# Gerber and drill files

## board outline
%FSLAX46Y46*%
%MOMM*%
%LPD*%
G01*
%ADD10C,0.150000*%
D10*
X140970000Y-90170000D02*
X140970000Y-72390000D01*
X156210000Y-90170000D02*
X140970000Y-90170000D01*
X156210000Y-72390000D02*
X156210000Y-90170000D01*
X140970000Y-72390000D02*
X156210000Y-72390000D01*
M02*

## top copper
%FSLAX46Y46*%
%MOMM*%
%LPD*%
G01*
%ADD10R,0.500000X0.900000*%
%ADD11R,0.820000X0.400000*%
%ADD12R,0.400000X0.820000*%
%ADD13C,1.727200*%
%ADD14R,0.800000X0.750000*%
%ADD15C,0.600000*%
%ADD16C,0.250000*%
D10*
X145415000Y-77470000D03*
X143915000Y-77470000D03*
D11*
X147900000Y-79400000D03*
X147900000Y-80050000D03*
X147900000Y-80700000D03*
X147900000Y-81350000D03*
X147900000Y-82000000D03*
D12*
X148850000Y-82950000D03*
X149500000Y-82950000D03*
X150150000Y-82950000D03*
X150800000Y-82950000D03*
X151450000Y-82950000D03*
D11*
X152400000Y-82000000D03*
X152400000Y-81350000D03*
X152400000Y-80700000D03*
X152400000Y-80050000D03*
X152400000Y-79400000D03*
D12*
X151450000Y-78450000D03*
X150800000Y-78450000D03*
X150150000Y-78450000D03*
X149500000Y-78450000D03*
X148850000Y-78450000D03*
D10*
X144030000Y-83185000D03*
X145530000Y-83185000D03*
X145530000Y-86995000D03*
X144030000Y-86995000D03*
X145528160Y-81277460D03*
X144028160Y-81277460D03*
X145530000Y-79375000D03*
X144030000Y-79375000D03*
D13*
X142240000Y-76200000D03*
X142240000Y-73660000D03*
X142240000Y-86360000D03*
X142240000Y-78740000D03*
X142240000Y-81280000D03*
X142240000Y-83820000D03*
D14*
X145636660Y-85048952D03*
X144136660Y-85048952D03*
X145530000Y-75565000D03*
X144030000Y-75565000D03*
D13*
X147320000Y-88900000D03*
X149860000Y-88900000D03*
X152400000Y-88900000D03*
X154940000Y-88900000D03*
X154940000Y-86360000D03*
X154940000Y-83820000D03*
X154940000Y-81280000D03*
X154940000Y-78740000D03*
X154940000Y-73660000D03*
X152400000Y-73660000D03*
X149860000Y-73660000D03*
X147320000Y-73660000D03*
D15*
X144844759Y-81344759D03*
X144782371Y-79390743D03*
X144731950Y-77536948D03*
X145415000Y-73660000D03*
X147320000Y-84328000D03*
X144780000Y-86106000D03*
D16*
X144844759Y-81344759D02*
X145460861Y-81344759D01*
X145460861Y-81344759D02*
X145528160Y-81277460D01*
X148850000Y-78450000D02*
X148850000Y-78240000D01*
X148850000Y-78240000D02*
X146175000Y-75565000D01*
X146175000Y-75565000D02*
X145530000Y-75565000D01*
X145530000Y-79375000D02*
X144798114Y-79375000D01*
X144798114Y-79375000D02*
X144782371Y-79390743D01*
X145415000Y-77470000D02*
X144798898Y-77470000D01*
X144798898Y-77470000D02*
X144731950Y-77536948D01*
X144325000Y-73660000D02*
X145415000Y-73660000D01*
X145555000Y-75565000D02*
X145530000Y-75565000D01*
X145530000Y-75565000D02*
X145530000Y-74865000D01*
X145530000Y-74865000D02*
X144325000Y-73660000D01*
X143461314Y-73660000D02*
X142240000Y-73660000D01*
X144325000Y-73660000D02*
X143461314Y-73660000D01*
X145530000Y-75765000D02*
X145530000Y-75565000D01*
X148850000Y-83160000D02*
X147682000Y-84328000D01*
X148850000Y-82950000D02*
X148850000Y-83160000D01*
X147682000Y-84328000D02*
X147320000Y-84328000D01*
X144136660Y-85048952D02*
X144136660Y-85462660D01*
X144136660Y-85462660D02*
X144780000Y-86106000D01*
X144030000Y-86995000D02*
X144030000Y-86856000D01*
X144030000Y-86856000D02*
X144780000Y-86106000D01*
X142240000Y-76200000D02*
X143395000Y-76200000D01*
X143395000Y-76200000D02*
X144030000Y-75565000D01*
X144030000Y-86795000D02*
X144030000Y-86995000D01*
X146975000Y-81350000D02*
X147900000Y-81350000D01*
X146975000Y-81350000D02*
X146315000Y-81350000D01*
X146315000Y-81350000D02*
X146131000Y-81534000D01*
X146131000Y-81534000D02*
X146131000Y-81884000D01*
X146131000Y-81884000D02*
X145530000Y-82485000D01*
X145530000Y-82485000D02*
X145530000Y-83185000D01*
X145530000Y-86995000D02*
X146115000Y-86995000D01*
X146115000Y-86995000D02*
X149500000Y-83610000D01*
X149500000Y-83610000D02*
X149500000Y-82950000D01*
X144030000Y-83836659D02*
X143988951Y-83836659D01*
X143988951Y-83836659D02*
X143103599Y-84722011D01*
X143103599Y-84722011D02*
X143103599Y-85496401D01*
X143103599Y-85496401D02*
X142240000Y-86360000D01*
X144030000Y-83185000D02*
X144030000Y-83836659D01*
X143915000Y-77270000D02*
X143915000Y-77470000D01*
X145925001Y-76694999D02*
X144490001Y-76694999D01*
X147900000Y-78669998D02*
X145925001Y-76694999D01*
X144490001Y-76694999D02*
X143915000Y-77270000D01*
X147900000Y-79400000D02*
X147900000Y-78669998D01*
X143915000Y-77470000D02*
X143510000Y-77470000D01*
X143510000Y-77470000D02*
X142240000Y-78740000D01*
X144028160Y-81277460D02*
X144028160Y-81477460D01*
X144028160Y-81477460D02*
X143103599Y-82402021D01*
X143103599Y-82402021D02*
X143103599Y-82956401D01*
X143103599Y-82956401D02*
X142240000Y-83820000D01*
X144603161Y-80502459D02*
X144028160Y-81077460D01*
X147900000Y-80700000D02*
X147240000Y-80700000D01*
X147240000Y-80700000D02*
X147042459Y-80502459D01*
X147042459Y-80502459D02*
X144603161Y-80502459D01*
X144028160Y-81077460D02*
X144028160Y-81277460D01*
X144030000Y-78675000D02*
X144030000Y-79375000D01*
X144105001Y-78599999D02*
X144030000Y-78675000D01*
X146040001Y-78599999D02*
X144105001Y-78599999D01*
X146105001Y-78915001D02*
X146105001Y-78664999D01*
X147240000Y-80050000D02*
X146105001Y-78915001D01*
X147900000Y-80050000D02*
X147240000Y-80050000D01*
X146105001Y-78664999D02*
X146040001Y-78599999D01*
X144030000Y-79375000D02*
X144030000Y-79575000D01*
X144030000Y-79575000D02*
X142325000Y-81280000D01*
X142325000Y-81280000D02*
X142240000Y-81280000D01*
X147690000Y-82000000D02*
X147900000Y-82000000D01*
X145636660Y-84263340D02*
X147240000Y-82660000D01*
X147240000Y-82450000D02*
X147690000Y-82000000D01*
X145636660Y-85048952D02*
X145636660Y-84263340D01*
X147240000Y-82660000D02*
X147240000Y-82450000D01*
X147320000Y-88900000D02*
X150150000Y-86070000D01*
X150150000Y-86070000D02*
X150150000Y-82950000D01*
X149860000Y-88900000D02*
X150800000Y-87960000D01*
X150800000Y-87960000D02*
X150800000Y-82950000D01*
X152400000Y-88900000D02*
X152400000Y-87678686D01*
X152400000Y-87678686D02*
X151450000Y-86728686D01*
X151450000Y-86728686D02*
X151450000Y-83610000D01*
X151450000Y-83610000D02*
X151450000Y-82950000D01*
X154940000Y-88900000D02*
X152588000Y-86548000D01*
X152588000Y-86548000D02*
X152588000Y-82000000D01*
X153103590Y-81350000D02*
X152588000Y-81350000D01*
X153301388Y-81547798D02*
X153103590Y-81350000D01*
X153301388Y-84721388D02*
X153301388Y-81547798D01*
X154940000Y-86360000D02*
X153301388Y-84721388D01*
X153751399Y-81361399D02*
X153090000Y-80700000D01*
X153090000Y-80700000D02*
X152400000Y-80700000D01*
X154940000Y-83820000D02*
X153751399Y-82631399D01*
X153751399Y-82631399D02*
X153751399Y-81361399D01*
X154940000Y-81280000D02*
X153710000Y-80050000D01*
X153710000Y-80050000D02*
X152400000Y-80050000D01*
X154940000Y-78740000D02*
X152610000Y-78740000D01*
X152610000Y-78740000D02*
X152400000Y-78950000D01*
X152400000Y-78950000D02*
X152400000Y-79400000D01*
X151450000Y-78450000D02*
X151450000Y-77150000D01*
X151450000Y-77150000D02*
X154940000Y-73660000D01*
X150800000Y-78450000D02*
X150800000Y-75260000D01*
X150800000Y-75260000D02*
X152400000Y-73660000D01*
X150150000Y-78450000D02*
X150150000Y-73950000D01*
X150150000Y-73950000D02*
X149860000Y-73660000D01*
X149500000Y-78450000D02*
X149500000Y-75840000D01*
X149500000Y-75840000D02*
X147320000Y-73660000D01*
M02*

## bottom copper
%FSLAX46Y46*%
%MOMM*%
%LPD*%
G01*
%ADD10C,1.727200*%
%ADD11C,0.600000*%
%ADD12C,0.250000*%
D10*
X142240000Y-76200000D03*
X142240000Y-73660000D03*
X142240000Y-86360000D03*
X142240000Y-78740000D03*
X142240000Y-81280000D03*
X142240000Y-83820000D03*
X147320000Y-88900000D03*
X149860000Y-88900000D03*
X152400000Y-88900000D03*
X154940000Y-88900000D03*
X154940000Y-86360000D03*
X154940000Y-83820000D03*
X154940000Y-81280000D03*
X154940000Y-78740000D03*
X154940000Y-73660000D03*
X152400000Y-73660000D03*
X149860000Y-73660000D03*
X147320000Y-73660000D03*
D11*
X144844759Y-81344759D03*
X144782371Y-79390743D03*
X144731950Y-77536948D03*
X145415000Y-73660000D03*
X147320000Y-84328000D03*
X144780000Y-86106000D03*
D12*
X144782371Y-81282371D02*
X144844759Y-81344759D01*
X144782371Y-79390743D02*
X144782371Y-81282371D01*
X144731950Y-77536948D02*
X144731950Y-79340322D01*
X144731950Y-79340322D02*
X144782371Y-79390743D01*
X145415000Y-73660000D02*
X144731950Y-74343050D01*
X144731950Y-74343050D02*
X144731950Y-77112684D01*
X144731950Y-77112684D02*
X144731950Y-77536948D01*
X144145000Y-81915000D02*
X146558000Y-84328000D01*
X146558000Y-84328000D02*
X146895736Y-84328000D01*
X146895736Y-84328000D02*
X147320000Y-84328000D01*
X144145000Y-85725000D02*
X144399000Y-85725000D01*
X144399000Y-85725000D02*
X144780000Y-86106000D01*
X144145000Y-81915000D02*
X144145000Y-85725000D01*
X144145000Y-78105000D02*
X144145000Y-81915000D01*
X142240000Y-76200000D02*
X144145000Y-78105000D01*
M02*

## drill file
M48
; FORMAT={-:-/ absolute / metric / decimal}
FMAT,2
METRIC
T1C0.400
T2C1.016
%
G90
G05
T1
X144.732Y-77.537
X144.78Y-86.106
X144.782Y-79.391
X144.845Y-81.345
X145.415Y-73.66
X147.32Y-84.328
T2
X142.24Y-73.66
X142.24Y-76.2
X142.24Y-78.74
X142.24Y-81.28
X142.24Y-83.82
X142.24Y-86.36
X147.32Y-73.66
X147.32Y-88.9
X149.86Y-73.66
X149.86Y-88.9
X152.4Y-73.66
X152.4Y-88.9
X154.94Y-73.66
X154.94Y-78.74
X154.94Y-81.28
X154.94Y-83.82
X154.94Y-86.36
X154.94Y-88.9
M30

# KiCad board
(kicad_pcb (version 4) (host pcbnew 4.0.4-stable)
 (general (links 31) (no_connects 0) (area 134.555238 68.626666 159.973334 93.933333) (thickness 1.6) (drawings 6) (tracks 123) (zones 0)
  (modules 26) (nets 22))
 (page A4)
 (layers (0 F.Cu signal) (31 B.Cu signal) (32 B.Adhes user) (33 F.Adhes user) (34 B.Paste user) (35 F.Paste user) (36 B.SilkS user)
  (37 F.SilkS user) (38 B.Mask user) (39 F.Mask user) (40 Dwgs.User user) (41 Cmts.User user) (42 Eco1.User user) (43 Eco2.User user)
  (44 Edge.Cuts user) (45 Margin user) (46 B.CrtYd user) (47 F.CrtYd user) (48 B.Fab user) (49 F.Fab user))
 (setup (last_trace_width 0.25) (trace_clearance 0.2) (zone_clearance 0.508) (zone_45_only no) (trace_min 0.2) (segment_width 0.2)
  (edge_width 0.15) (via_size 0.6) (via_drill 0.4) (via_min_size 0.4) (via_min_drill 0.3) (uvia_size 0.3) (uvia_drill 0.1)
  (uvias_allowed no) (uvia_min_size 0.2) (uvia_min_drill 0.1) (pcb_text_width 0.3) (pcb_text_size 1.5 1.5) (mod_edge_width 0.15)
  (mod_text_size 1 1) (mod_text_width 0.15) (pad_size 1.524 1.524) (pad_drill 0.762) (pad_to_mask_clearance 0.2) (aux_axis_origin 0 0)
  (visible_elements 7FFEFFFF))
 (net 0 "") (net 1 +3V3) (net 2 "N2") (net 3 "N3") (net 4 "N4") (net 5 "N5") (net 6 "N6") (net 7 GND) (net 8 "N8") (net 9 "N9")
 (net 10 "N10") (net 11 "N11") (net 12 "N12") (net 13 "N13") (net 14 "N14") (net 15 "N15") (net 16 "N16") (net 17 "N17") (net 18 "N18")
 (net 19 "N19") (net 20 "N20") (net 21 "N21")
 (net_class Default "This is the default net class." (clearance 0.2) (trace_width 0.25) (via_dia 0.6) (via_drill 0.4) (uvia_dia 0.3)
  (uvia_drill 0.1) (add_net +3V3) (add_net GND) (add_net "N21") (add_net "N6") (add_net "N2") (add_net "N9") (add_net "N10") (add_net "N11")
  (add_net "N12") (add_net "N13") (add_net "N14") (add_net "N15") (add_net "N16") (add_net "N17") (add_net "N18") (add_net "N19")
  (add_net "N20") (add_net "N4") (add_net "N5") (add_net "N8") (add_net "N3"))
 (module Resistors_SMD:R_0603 (layer F.Cu) (at 144.665 77.47 180)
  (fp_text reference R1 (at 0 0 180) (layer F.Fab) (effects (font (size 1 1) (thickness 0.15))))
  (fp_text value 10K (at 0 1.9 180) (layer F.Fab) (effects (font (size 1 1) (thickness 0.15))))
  (pad 1 smd rect (at -0.75 0 180) (size 0.5 0.9) (layers F.Cu F.Paste F.Mask) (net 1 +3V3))
  (pad 2 smd rect (at 0.75 0 180) (size 0.5 0.9) (layers F.Cu F.Paste F.Mask) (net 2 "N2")))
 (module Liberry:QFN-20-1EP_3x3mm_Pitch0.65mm (layer F.Cu) (at 150.15 80.7)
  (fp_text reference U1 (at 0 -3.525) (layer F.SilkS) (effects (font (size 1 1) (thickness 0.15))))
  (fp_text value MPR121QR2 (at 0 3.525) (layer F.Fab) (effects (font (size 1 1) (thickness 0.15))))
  (pad 1 smd rect (at -2.25 -1.3) (size 0.82 0.4) (layers F.Cu F.Paste F.Mask) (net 2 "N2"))
  (pad 2 smd rect (at -2.25 -0.65) (size 0.82 0.4) (layers F.Cu F.Paste F.Mask) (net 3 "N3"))
  (pad 3 smd rect (at -2.25 0) (size 0.82 0.4) (layers F.Cu F.Paste F.Mask) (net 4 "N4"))
  (pad 4 smd rect (at -2.25 0.65) (size 0.82 0.4) (layers F.Cu F.Paste F.Mask) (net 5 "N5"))
  (pad 5 smd rect (at -2.25 1.3) (size 0.82 0.4) (layers F.Cu F.Paste F.Mask) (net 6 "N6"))
  (pad 6 smd rect (at -1.3 2.25 90) (size 0.82 0.4) (layers F.Cu F.Paste F.Mask) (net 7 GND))
  (pad 7 smd rect (at -0.65 2.25 90) (size 0.82 0.4) (layers F.Cu F.Paste F.Mask) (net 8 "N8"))
  (pad 8 smd rect (at 0 2.25 90) (size 0.82 0.4) (layers F.Cu F.Paste F.Mask) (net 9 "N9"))
  (pad 9 smd rect (at 0.65 2.25 90) (size 0.82 0.4) (layers F.Cu F.Paste F.Mask) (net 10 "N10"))
  (pad 10 smd rect (at 1.3 2.25 90) (size 0.82 0.4) (layers F.Cu F.Paste F.Mask) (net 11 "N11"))
  (pad 11 smd rect (at 2.25 1.3) (size 0.82 0.4) (layers F.Cu F.Paste F.Mask) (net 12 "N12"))
  (pad 12 smd rect (at 2.25 0.65) (size 0.82 0.4) (layers F.Cu F.Paste F.Mask) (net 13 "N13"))
  (pad 13 smd rect (at 2.25 0) (size 0.82 0.4) (layers F.Cu F.Paste F.Mask) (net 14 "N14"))
  (pad 14 smd rect (at 2.25 -0.65) (size 0.82 0.4) (layers F.Cu F.Paste F.Mask) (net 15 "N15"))
  (pad 15 smd rect (at 2.25 -1.3) (size 0.82 0.4) (layers F.Cu F.Paste F.Mask) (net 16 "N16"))
  (pad 16 smd rect (at 1.3 -2.25 90) (size 0.82 0.4) (layers F.Cu F.Paste F.Mask) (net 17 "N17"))
  (pad 17 smd rect (at 0.65 -2.25 90) (size 0.82 0.4) (layers F.Cu F.Paste F.Mask) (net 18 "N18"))
  (pad 18 smd rect (at 0 -2.25 90) (size 0.82 0.4) (layers F.Cu F.Paste F.Mask) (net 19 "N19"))
  (pad 19 smd rect (at -0.65 -2.25 90) (size 0.82 0.4) (layers F.Cu F.Paste F.Mask) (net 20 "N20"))
  (pad 20 smd rect (at -1.3 -2.25 90) (size 0.82 0.4) (layers F.Cu F.Paste F.Mask) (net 1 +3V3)))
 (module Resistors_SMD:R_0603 (layer F.Cu) (at 144.78 83.185)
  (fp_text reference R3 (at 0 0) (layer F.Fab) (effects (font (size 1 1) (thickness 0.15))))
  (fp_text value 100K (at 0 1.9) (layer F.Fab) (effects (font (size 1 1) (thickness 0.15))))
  (pad 1 smd rect (at -0.75 0) (size 0.5 0.9) (layers F.Cu F.Paste F.Mask) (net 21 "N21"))
  (pad 2 smd rect (at 0.75 0) (size 0.5 0.9) (layers F.Cu F.Paste F.Mask) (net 5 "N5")))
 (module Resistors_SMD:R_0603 (layer F.Cu) (at 144.78 86.995 180)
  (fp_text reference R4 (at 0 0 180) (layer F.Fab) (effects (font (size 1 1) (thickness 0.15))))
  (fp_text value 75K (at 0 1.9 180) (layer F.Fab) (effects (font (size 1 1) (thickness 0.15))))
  (pad 1 smd rect (at -0.75 0 180) (size 0.5 0.9) (layers F.Cu F.Paste F.Mask) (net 8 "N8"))
  (pad 2 smd rect (at 0.75 0 180) (size 0.5 0.9) (layers F.Cu F.Paste F.Mask) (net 7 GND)))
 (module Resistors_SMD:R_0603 (layer F.Cu) (at 144.77816 81.27746 180)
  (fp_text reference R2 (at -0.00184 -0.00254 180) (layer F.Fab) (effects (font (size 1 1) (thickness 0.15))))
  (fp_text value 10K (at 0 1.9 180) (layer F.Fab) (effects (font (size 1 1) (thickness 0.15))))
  (pad 1 smd rect (at -0.75 0 180) (size 0.5 0.9) (layers F.Cu F.Paste F.Mask) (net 1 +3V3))
  (pad 2 smd rect (at 0.75 0 180) (size 0.5 0.9) (layers F.Cu F.Paste F.Mask) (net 4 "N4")))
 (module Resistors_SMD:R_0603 (layer F.Cu) (at 144.78 79.375 180)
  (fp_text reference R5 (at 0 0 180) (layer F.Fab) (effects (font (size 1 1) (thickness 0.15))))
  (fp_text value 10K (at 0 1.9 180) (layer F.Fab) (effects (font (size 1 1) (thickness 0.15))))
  (pad 1 smd rect (at -0.75 0 180) (size 0.5 0.9) (layers F.Cu F.Paste F.Mask) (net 1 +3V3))
  (pad 2 smd rect (at 0.75 0 180) (size 0.5 0.9) (layers F.Cu F.Paste F.Mask) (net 3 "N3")))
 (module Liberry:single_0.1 (layer F.Cu) (at 142.24 76.2)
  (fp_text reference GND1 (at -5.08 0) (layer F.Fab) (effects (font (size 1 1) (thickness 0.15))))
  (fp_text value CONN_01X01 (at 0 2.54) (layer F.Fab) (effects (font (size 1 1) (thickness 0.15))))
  (pad 1 thru_hole circle (at 0 0) (size 1.7272 1.7272) (drill 1.016) (layers *.Cu *.Mask) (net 7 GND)))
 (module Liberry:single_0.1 (layer F.Cu) (at 142.24 73.66)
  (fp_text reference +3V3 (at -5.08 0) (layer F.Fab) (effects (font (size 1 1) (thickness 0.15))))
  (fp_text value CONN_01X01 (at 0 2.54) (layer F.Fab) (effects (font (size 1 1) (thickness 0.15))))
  (pad 1 thru_hole circle (at 0 0) (size 1.7272 1.7272) (drill 1.016) (layers *.Cu *.Mask) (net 1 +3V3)))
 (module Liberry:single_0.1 (layer F.Cu) (at 142.24 86.36)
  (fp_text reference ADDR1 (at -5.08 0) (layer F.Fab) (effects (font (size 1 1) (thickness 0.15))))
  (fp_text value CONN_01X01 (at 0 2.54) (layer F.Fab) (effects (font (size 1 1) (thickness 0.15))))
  (pad 1 thru_hole circle (at 0 0) (size 1.7272 1.7272) (drill 1.016) (layers *.Cu *.Mask) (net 21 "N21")))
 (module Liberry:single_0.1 (layer F.Cu) (at 142.24 78.74)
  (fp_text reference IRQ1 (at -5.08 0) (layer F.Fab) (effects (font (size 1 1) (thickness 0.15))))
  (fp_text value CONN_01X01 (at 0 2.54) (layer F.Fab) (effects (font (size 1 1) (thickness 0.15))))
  (pad 1 thru_hole circle (at 0 0) (size 1.7272 1.7272) (drill 1.016) (layers *.Cu *.Mask) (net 2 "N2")))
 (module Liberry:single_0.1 (layer F.Cu) (at 142.24 81.28)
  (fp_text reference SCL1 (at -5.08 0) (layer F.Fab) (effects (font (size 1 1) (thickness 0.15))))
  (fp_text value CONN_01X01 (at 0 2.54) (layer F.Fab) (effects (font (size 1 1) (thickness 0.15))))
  (pad 1 thru_hole circle (at 0 0) (size 1.7272 1.7272) (drill 1.016) (layers *.Cu *.Mask) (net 3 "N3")))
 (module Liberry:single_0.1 (layer F.Cu) (at 142.24 83.82)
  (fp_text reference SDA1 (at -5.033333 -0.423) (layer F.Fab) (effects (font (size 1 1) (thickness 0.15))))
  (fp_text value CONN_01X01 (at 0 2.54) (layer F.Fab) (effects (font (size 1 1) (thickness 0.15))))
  (pad 1 thru_hole circle (at 0 0) (size 1.7272 1.7272) (drill 1.016) (layers *.Cu *.Mask) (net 4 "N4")))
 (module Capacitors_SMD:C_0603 (layer F.Cu) (at 144.88666 85.048952 180)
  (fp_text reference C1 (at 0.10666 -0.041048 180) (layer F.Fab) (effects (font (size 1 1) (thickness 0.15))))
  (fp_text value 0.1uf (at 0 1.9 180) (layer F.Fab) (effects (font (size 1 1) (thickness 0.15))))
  (pad 1 smd rect (at -0.75 0 180) (size 0.8 0.75) (layers F.Cu F.Paste F.Mask) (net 6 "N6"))
  (pad 2 smd rect (at 0.75 0 180) (size 0.8 0.75) (layers F.Cu F.Paste F.Mask) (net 7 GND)))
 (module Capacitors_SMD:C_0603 (layer F.Cu) (at 144.78 75.565 180)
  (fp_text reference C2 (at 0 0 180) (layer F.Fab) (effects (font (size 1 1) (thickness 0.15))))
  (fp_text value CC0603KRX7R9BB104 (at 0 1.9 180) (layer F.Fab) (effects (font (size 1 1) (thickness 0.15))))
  (pad 1 smd rect (at -0.75 0 180) (size 0.8 0.75) (layers F.Cu F.Paste F.Mask) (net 1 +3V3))
  (pad 2 smd rect (at 0.75 0 180) (size 0.8 0.75) (layers F.Cu F.Paste F.Mask) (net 7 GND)))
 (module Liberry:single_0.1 (layer F.Cu) (at 147.32 88.9 270)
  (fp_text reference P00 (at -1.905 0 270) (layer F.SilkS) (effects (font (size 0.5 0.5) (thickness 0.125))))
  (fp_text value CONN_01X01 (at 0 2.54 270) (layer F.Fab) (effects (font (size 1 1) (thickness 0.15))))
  (pad 1 thru_hole circle (at 0 0 270) (size 1.7272 1.7272) (drill 1.016) (layers *.Cu *.Mask) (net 9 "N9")))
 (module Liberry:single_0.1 (layer F.Cu) (at 149.86 88.9 270)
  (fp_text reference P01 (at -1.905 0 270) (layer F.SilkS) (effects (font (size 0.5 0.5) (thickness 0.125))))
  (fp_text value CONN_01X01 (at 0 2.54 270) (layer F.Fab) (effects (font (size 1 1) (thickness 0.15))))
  (pad 1 thru_hole circle (at 0 0 270) (size 1.7272 1.7272) (drill 1.016) (layers *.Cu *.Mask) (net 10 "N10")))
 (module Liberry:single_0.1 (layer F.Cu) (at 152.4 88.9 270)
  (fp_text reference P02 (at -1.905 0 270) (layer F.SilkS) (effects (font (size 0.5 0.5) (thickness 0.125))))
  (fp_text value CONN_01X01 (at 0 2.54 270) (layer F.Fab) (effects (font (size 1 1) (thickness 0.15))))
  (pad 1 thru_hole circle (at 0 0 270) (size 1.7272 1.7272) (drill 1.016) (layers *.Cu *.Mask) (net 11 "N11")))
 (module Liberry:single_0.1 (layer F.Cu) (at 154.94 88.9 270)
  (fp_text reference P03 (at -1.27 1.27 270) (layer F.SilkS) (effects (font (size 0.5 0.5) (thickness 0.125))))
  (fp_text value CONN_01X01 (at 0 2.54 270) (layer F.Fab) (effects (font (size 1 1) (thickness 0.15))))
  (pad 1 thru_hole circle (at 0 0 270) (size 1.7272 1.7272) (drill 1.016) (layers *.Cu *.Mask) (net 12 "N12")))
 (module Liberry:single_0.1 (layer F.Cu) (at 154.94 86.36)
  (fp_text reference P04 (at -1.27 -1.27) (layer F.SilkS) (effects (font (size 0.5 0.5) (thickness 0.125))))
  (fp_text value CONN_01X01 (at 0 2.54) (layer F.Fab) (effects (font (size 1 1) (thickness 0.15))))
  (pad 1 thru_hole circle (at 0 0) (size 1.7272 1.7272) (drill 1.016) (layers *.Cu *.Mask) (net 13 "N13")))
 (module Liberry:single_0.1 (layer F.Cu) (at 154.94 83.82)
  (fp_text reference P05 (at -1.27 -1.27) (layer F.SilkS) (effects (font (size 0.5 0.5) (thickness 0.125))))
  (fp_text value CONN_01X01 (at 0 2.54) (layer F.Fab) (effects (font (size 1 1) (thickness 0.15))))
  (pad 1 thru_hole circle (at 0 0) (size 1.7272 1.7272) (drill 1.016) (layers *.Cu *.Mask) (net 14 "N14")))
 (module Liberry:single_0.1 (layer F.Cu) (at 154.94 81.28)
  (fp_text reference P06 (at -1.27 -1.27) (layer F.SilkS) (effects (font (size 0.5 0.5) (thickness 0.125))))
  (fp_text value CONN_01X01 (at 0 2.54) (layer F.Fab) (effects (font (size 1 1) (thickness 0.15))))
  (pad 1 thru_hole circle (at 0 0) (size 1.7272 1.7272) (drill 1.016) (layers *.Cu *.Mask) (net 15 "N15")))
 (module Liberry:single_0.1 (layer F.Cu) (at 154.94 78.74)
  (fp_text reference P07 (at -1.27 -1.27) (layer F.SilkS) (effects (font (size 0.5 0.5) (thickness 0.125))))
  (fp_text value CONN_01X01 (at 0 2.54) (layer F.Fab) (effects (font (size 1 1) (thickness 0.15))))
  (pad 1 thru_hole circle (at 0 0) (size 1.7272 1.7272) (drill 1.016) (layers *.Cu *.Mask) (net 16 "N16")))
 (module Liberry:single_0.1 (layer F.Cu) (at 154.94 73.66 90)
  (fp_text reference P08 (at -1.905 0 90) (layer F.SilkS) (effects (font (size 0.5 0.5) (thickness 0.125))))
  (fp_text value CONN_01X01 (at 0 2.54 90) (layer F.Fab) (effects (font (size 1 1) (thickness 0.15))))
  (pad 1 thru_hole circle (at 0 0 90) (size 1.7272 1.7272) (drill 1.016) (layers *.Cu *.Mask) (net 17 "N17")))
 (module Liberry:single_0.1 (layer F.Cu) (at 152.4 73.66 90)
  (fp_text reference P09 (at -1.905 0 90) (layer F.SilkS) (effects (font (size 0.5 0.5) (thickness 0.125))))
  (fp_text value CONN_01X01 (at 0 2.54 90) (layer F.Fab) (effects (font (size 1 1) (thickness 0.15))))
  (pad 1 thru_hole circle (at 0 0 90) (size 1.7272 1.7272) (drill 1.016) (layers *.Cu *.Mask) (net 18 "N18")))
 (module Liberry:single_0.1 (layer F.Cu) (at 149.86 73.66 90)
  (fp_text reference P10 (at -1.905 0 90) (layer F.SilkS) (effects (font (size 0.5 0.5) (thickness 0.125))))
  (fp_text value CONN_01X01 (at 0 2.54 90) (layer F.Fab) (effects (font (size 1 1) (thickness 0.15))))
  (pad 1 thru_hole circle (at 0 0 90) (size 1.7272 1.7272) (drill 1.016) (layers *.Cu *.Mask) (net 19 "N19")))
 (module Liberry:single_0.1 (layer F.Cu) (at 147.32 73.66 90)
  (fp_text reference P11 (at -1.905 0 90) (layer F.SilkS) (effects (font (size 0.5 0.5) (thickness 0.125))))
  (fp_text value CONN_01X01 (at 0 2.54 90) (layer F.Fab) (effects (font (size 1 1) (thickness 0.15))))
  (pad 1 thru_hole circle (at 0 0 90) (size 1.7272 1.7272) (drill 1.016) (layers *.Cu *.Mask) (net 20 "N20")))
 (gr_line (start 140.97 90.17) (end 140.97 72.39) (layer Edge.Cuts) (width 0.15))
 (gr_line (start 156.21 90.17) (end 140.97 90.17) (layer Edge.Cuts) (width 0.15))
 (gr_line (start 156.21 72.39) (end 156.21 90.17) (layer Edge.Cuts) (width 0.15))
 (gr_line (start 140.97 72.39) (end 156.21 72.39) (layer Edge.Cuts) (width 0.15))
 (segment (start 144.844759 81.344759) (end 145.460861 81.344759) (width 0.25) (layer F.Cu) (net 1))
 (segment (start 145.460861 81.344759) (end 145.52816 81.27746) (width 0.25) (layer F.Cu) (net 1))
 (segment (start 148.85 78.45) (end 148.85 78.24) (width 0.25) (layer F.Cu) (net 1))
 (segment (start 148.85 78.24) (end 146.175 75.565) (width 0.25) (layer F.Cu) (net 1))
 (segment (start 146.175 75.565) (end 145.53 75.565) (width 0.25) (layer F.Cu) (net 1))
 (segment (start 144.782371 81.282371) (end 144.844759 81.344759) (width 0.25) (layer B.Cu) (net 1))
 (segment (start 144.782371 79.390743) (end 144.782371 81.282371) (width 0.25) (layer B.Cu) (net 1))
 (via (at 144.844759 81.344759) (size 0.6) (drill 0.4) (layers F.Cu B.Cu) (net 1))
 (segment (start 145.53 79.375) (end 144.798114 79.375) (width 0.25) (layer F.Cu) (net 1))
 (segment (start 144.73195 77.536948) (end 144.73195 79.340322) (width 0.25) (layer B.Cu) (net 1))
 (segment (start 144.73195 79.340322) (end 144.782371 79.390743) (width 0.25) (layer B.Cu) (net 1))
 (segment (start 144.798114 79.375) (end 144.782371 79.390743) (width 0.25) (layer F.Cu) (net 1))
 (via (at 144.782371 79.390743) (size 0.6) (drill 0.4) (layers F.Cu B.Cu) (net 1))
 (via (at 144.73195 77.536948) (size 0.6) (drill 0.4) (layers F.Cu B.Cu) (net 1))
 (segment (start 145.415 77.47) (end 144.798898 77.47) (width 0.25) (layer F.Cu) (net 1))
 (segment (start 144.798898 77.47) (end 144.73195 77.536948) (width 0.25) (layer F.Cu) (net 1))
 (segment (start 145.415 73.66) (end 144.73195 74.34305) (width 0.25) (layer B.Cu) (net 1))
 (segment (start 144.73195 74.34305) (end 144.73195 77.112684) (width 0.25) (layer B.Cu) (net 1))
 (segment (start 144.73195 77.112684) (end 144.73195 77.536948) (width 0.25) (layer B.Cu) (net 1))
 (segment (start 144.325 73.66) (end 145.415 73.66) (width 0.25) (layer F.Cu) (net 1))
 (via (at 145.415 73.66) (size 0.6) (drill 0.4) (layers F.Cu B.Cu) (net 1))
 (segment (start 145.555 75.565) (end 145.53 75.565) (width 0.25) (layer F.Cu) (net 1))
 (segment (start 145.53 75.565) (end 145.53 74.865) (width 0.25) (layer F.Cu) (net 1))
 (segment (start 145.53 74.865) (end 144.325 73.66) (width 0.25) (layer F.Cu) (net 1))
 (segment (start 143.461314 73.66) (end 142.24 73.66) (width 0.25) (layer F.Cu) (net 1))
 (segment (start 144.325 73.66) (end 143.461314 73.66) (width 0.25) (layer F.Cu) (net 1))
 (segment (start 145.53 75.765) (end 145.53 75.565) (width 0.25) (layer F.Cu) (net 1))
 (segment (start 144.145 81.915) (end 146.558 84.328) (width 0.25) (layer B.Cu) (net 7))
 (segment (start 146.558 84.328) (end 146.895736 84.328) (width 0.25) (layer B.Cu) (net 7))
 (segment (start 146.895736 84.328) (end 147.32 84.328) (width 0.25) (layer B.Cu) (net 7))
 (segment (start 148.85 83.16) (end 147.682 84.328) (width 0.25) (layer F.Cu) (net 7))
 (segment (start 148.85 82.95) (end 148.85 83.16) (width 0.25) (layer F.Cu) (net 7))
 (segment (start 147.682 84.328) (end 147.32 84.328) (width 0.25) (layer F.Cu) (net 7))
 (via (at 147.32 84.328) (size 0.6) (drill 0.4) (layers F.Cu B.Cu) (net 7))
 (segment (start 144.13666 85.048952) (end 144.13666 85.46266) (width 0.25) (layer F.Cu) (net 7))
 (segment (start 144.13666 85.46266) (end 144.78 86.106) (width 0.25) (layer F.Cu) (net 7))
 (segment (start 144.03 86.995) (end 144.03 86.856) (width 0.25) (layer F.Cu) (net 7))
 (segment (start 144.03 86.856) (end 144.78 86.106) (width 0.25) (layer F.Cu) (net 7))
 (segment (start 144.145 85.725) (end 144.399 85.725) (width 0.25) (layer B.Cu) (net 7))
 (segment (start 144.399 85.725) (end 144.78 86.106) (width 0.25) (layer B.Cu) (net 7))
 (segment (start 144.145 81.915) (end 144.145 85.725) (width 0.25) (layer B.Cu) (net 7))
 (via (at 144.78 86.106) (size 0.6) (drill 0.4) (layers F.Cu B.Cu) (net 7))
 (segment (start 144.145 78.105) (end 144.145 81.915) (width 0.25) (layer B.Cu) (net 7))
 (segment (start 142.24 76.2) (end 144.145 78.105) (width 0.25) (layer B.Cu) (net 7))
 (segment (start 142.24 76.2) (end 143.395 76.2) (width 0.25) (layer F.Cu) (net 7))
 (segment (start 143.395 76.2) (end 144.03 75.565) (width 0.25) (layer F.Cu) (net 7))
 (segment (start 144.03 86.795) (end 144.03 86.995) (width 0.25) (layer F.Cu) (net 7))
 (segment (start 146.975 81.35) (end 147.9 81.35) (width 0.25) (layer F.Cu) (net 5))
 (segment (start 146.975 81.35) (end 146.315 81.35) (width 0.25) (layer F.Cu) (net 5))
 (segment (start 146.315 81.35) (end 146.131 81.534) (width 0.25) (layer F.Cu) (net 5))
 (segment (start 146.131 81.534) (end 146.131 81.884) (width 0.25) (layer F.Cu) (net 5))
 (segment (start 146.131 81.884) (end 145.53 82.485) (width 0.25) (layer F.Cu) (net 5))
 (segment (start 145.53 82.485) (end 145.53 83.185) (width 0.25) (layer F.Cu) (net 5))
 (segment (start 145.53 86.995) (end 146.115 86.995) (width 0.25) (layer F.Cu) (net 8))
 (segment (start 146.115 86.995) (end 149.5 83.61) (width 0.25) (layer F.Cu) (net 8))
 (segment (start 149.5 83.61) (end 149.5 82.95) (width 0.25) (layer F.Cu) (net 8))
 (segment (start 144.03 83.836659) (end 143.988951 83.836659) (width 0.25) (layer F.Cu) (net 21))
 (segment (start 143.988951 83.836659) (end 143.103599 84.722011) (width 0.25) (layer F.Cu) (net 21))
 (segment (start 143.103599 84.722011) (end 143.103599 85.496401) (width 0.25) (layer F.Cu) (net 21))
 (segment (start 143.103599 85.496401) (end 142.24 86.36) (width 0.25) (layer F.Cu) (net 21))
 (segment (start 144.03 83.185) (end 144.03 83.836659) (width 0.25) (layer F.Cu) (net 21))
 (segment (start 143.915 77.27) (end 143.915 77.47) (width 0.25) (layer F.Cu) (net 2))
 (segment (start 145.925001 76.694999) (end 144.490001 76.694999) (width 0.25) (layer F.Cu) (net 2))
 (segment (start 147.9 78.669998) (end 145.925001 76.694999) (width 0.25) (layer F.Cu) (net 2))
 (segment (start 144.490001 76.694999) (end 143.915 77.27) (width 0.25) (layer F.Cu) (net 2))
 (segment (start 147.9 79.4) (end 147.9 78.669998) (width 0.25) (layer F.Cu) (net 2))
 (segment (start 143.915 77.47) (end 143.51 77.47) (width 0.25) (layer F.Cu) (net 2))
 (segment (start 143.51 77.47) (end 142.24 78.74) (width 0.25) (layer F.Cu) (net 2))
 (segment (start 144.02816 81.27746) (end 144.02816 81.47746) (width 0.25) (layer F.Cu) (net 4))
 (segment (start 144.02816 81.47746) (end 143.103599 82.402021) (width 0.25) (layer F.Cu) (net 4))
 (segment (start 143.103599 82.402021) (end 143.103599 82.956401) (width 0.25) (layer F.Cu) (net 4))
 (segment (start 143.103599 82.956401) (end 142.24 83.82) (width 0.25) (layer F.Cu) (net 4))
 (segment (start 144.603161 80.502459) (end 144.02816 81.07746) (width 0.25) (layer F.Cu) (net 4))
 (segment (start 147.9 80.7) (end 147.24 80.7) (width 0.25) (layer F.Cu) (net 4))
 (segment (start 147.24 80.7) (end 147.042459 80.502459) (width 0.25) (layer F.Cu) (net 4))
 (segment (start 147.042459 80.502459) (end 144.603161 80.502459) (width 0.25) (layer F.Cu) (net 4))
 (segment (start 144.02816 81.07746) (end 144.02816 81.27746) (width 0.25) (layer F.Cu) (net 4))
 (segment (start 144.03 78.675) (end 144.03 79.375) (width 0.25) (layer F.Cu) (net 3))
 (segment (start 144.105001 78.599999) (end 144.03 78.675) (width 0.25) (layer F.Cu) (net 3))
 (segment (start 146.040001 78.599999) (end 144.105001 78.599999) (width 0.25) (layer F.Cu) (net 3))
 (segment (start 146.105001 78.915001) (end 146.105001 78.664999) (width 0.25) (layer F.Cu) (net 3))
 (segment (start 147.24 80.05) (end 146.105001 78.915001) (width 0.25) (layer F.Cu) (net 3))
 (segment (start 147.9 80.05) (end 147.24 80.05) (width 0.25) (layer F.Cu) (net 3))
 (segment (start 146.105001 78.664999) (end 146.040001 78.599999) (width 0.25) (layer F.Cu) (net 3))
 (segment (start 144.03 79.375) (end 144.03 79.575) (width 0.25) (layer F.Cu) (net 3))
 (segment (start 144.03 79.575) (end 142.325 81.28) (width 0.25) (layer F.Cu) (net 3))
 (segment (start 142.325 81.28) (end 142.24 81.28) (width 0.25) (layer F.Cu) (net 3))
 (segment (start 147.69 82) (end 147.9 82) (width 0.25) (layer F.Cu) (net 6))
 (segment (start 145.63666 84.26334) (end 147.24 82.66) (width 0.25) (layer F.Cu) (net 6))
 (segment (start 147.24 82.45) (end 147.69 82) (width 0.25) (layer F.Cu) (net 6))
 (segment (start 145.63666 85.048952) (end 145.63666 84.26334) (width 0.25) (layer F.Cu) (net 6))
 (segment (start 147.24 82.66) (end 147.24 82.45) (width 0.25) (layer F.Cu) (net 6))
 (segment (start 147.32 88.9) (end 150.15 86.07) (width 0.25) (layer F.Cu) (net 9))
 (segment (start 150.15 86.07) (end 150.15 82.95) (width 0.25) (layer F.Cu) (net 9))
 (segment (start 149.86 88.9) (end 150.8 87.96) (width 0.25) (layer F.Cu) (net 10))
 (segment (start 150.8 87.96) (end 150.8 82.95) (width 0.25) (layer F.Cu) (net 10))
 (segment (start 152.4 88.9) (end 152.4 87.678686) (width 0.25) (layer F.Cu) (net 11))
 (segment (start 152.4 87.678686) (end 151.45 86.728686) (width 0.25) (layer F.Cu) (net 11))
 (segment (start 151.45 86.728686) (end 151.45 83.61) (width 0.25) (layer F.Cu) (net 11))
 (segment (start 151.45 83.61) (end 151.45 82.95) (width 0.25) (layer F.Cu) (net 11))
 (segment (start 154.94 88.9) (end 152.588 86.548) (width 0.25) (layer F.Cu) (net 12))
 (segment (start 152.588 86.548) (end 152.588 82) (width 0.25) (layer F.Cu) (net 12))
 (segment (start 153.10359 81.35) (end 152.588 81.35) (width 0.25) (layer F.Cu) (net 13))
 (segment (start 153.301388 81.547798) (end 153.10359 81.35) (width 0.25) (layer F.Cu) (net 13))
 (segment (start 153.301388 84.721388) (end 153.301388 81.547798) (width 0.25) (layer F.Cu) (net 13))
 (segment (start 154.94 86.36) (end 153.301388 84.721388) (width 0.25) (layer F.Cu) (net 13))
 (segment (start 153.751399 81.361399) (end 153.09 80.7) (width 0.25) (layer F.Cu) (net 14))
 (segment (start 153.09 80.7) (end 152.4 80.7) (width 0.25) (layer F.Cu) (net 14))
 (segment (start 154.94 83.82) (end 153.751399 82.631399) (width 0.25) (layer F.Cu) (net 14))
 (segment (start 153.751399 82.631399) (end 153.751399 81.361399) (width 0.25) (layer F.Cu) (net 14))
 (segment (start 154.94 81.28) (end 153.71 80.05) (width 0.25) (layer F.Cu) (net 15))
 (segment (start 153.71 80.05) (end 152.4 80.05) (width 0.25) (layer F.Cu) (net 15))
 (segment (start 154.94 78.74) (end 152.61 78.74) (width 0.25) (layer F.Cu) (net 16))
 (segment (start 152.61 78.74) (end 152.4 78.95) (width 0.25) (layer F.Cu) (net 16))
 (segment (start 152.4 78.95) (end 152.4 79.4) (width 0.25) (layer F.Cu) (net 16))
 (segment (start 151.45 78.45) (end 151.45 77.15) (width 0.25) (layer F.Cu) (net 17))
 (segment (start 151.45 77.15) (end 154.94 73.66) (width 0.25) (layer F.Cu) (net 17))
 (segment (start 150.8 78.45) (end 150.8 75.26) (width 0.25) (layer F.Cu) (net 18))
 (segment (start 150.8 75.26) (end 152.4 73.66) (width 0.25) (layer F.Cu) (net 18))
 (segment (start 150.15 78.45) (end 150.15 73.95) (width 0.25) (layer F.Cu) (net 19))
 (segment (start 150.15 73.95) (end 149.86 73.66) (width 0.25) (layer F.Cu) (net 19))
 (segment (start 149.5 78.45) (end 149.5 75.84) (width 0.25) (layer F.Cu) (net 20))
 (segment (start 149.5 75.84) (end 147.32 73.66) (width 0.25) (layer F.Cu) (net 20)))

